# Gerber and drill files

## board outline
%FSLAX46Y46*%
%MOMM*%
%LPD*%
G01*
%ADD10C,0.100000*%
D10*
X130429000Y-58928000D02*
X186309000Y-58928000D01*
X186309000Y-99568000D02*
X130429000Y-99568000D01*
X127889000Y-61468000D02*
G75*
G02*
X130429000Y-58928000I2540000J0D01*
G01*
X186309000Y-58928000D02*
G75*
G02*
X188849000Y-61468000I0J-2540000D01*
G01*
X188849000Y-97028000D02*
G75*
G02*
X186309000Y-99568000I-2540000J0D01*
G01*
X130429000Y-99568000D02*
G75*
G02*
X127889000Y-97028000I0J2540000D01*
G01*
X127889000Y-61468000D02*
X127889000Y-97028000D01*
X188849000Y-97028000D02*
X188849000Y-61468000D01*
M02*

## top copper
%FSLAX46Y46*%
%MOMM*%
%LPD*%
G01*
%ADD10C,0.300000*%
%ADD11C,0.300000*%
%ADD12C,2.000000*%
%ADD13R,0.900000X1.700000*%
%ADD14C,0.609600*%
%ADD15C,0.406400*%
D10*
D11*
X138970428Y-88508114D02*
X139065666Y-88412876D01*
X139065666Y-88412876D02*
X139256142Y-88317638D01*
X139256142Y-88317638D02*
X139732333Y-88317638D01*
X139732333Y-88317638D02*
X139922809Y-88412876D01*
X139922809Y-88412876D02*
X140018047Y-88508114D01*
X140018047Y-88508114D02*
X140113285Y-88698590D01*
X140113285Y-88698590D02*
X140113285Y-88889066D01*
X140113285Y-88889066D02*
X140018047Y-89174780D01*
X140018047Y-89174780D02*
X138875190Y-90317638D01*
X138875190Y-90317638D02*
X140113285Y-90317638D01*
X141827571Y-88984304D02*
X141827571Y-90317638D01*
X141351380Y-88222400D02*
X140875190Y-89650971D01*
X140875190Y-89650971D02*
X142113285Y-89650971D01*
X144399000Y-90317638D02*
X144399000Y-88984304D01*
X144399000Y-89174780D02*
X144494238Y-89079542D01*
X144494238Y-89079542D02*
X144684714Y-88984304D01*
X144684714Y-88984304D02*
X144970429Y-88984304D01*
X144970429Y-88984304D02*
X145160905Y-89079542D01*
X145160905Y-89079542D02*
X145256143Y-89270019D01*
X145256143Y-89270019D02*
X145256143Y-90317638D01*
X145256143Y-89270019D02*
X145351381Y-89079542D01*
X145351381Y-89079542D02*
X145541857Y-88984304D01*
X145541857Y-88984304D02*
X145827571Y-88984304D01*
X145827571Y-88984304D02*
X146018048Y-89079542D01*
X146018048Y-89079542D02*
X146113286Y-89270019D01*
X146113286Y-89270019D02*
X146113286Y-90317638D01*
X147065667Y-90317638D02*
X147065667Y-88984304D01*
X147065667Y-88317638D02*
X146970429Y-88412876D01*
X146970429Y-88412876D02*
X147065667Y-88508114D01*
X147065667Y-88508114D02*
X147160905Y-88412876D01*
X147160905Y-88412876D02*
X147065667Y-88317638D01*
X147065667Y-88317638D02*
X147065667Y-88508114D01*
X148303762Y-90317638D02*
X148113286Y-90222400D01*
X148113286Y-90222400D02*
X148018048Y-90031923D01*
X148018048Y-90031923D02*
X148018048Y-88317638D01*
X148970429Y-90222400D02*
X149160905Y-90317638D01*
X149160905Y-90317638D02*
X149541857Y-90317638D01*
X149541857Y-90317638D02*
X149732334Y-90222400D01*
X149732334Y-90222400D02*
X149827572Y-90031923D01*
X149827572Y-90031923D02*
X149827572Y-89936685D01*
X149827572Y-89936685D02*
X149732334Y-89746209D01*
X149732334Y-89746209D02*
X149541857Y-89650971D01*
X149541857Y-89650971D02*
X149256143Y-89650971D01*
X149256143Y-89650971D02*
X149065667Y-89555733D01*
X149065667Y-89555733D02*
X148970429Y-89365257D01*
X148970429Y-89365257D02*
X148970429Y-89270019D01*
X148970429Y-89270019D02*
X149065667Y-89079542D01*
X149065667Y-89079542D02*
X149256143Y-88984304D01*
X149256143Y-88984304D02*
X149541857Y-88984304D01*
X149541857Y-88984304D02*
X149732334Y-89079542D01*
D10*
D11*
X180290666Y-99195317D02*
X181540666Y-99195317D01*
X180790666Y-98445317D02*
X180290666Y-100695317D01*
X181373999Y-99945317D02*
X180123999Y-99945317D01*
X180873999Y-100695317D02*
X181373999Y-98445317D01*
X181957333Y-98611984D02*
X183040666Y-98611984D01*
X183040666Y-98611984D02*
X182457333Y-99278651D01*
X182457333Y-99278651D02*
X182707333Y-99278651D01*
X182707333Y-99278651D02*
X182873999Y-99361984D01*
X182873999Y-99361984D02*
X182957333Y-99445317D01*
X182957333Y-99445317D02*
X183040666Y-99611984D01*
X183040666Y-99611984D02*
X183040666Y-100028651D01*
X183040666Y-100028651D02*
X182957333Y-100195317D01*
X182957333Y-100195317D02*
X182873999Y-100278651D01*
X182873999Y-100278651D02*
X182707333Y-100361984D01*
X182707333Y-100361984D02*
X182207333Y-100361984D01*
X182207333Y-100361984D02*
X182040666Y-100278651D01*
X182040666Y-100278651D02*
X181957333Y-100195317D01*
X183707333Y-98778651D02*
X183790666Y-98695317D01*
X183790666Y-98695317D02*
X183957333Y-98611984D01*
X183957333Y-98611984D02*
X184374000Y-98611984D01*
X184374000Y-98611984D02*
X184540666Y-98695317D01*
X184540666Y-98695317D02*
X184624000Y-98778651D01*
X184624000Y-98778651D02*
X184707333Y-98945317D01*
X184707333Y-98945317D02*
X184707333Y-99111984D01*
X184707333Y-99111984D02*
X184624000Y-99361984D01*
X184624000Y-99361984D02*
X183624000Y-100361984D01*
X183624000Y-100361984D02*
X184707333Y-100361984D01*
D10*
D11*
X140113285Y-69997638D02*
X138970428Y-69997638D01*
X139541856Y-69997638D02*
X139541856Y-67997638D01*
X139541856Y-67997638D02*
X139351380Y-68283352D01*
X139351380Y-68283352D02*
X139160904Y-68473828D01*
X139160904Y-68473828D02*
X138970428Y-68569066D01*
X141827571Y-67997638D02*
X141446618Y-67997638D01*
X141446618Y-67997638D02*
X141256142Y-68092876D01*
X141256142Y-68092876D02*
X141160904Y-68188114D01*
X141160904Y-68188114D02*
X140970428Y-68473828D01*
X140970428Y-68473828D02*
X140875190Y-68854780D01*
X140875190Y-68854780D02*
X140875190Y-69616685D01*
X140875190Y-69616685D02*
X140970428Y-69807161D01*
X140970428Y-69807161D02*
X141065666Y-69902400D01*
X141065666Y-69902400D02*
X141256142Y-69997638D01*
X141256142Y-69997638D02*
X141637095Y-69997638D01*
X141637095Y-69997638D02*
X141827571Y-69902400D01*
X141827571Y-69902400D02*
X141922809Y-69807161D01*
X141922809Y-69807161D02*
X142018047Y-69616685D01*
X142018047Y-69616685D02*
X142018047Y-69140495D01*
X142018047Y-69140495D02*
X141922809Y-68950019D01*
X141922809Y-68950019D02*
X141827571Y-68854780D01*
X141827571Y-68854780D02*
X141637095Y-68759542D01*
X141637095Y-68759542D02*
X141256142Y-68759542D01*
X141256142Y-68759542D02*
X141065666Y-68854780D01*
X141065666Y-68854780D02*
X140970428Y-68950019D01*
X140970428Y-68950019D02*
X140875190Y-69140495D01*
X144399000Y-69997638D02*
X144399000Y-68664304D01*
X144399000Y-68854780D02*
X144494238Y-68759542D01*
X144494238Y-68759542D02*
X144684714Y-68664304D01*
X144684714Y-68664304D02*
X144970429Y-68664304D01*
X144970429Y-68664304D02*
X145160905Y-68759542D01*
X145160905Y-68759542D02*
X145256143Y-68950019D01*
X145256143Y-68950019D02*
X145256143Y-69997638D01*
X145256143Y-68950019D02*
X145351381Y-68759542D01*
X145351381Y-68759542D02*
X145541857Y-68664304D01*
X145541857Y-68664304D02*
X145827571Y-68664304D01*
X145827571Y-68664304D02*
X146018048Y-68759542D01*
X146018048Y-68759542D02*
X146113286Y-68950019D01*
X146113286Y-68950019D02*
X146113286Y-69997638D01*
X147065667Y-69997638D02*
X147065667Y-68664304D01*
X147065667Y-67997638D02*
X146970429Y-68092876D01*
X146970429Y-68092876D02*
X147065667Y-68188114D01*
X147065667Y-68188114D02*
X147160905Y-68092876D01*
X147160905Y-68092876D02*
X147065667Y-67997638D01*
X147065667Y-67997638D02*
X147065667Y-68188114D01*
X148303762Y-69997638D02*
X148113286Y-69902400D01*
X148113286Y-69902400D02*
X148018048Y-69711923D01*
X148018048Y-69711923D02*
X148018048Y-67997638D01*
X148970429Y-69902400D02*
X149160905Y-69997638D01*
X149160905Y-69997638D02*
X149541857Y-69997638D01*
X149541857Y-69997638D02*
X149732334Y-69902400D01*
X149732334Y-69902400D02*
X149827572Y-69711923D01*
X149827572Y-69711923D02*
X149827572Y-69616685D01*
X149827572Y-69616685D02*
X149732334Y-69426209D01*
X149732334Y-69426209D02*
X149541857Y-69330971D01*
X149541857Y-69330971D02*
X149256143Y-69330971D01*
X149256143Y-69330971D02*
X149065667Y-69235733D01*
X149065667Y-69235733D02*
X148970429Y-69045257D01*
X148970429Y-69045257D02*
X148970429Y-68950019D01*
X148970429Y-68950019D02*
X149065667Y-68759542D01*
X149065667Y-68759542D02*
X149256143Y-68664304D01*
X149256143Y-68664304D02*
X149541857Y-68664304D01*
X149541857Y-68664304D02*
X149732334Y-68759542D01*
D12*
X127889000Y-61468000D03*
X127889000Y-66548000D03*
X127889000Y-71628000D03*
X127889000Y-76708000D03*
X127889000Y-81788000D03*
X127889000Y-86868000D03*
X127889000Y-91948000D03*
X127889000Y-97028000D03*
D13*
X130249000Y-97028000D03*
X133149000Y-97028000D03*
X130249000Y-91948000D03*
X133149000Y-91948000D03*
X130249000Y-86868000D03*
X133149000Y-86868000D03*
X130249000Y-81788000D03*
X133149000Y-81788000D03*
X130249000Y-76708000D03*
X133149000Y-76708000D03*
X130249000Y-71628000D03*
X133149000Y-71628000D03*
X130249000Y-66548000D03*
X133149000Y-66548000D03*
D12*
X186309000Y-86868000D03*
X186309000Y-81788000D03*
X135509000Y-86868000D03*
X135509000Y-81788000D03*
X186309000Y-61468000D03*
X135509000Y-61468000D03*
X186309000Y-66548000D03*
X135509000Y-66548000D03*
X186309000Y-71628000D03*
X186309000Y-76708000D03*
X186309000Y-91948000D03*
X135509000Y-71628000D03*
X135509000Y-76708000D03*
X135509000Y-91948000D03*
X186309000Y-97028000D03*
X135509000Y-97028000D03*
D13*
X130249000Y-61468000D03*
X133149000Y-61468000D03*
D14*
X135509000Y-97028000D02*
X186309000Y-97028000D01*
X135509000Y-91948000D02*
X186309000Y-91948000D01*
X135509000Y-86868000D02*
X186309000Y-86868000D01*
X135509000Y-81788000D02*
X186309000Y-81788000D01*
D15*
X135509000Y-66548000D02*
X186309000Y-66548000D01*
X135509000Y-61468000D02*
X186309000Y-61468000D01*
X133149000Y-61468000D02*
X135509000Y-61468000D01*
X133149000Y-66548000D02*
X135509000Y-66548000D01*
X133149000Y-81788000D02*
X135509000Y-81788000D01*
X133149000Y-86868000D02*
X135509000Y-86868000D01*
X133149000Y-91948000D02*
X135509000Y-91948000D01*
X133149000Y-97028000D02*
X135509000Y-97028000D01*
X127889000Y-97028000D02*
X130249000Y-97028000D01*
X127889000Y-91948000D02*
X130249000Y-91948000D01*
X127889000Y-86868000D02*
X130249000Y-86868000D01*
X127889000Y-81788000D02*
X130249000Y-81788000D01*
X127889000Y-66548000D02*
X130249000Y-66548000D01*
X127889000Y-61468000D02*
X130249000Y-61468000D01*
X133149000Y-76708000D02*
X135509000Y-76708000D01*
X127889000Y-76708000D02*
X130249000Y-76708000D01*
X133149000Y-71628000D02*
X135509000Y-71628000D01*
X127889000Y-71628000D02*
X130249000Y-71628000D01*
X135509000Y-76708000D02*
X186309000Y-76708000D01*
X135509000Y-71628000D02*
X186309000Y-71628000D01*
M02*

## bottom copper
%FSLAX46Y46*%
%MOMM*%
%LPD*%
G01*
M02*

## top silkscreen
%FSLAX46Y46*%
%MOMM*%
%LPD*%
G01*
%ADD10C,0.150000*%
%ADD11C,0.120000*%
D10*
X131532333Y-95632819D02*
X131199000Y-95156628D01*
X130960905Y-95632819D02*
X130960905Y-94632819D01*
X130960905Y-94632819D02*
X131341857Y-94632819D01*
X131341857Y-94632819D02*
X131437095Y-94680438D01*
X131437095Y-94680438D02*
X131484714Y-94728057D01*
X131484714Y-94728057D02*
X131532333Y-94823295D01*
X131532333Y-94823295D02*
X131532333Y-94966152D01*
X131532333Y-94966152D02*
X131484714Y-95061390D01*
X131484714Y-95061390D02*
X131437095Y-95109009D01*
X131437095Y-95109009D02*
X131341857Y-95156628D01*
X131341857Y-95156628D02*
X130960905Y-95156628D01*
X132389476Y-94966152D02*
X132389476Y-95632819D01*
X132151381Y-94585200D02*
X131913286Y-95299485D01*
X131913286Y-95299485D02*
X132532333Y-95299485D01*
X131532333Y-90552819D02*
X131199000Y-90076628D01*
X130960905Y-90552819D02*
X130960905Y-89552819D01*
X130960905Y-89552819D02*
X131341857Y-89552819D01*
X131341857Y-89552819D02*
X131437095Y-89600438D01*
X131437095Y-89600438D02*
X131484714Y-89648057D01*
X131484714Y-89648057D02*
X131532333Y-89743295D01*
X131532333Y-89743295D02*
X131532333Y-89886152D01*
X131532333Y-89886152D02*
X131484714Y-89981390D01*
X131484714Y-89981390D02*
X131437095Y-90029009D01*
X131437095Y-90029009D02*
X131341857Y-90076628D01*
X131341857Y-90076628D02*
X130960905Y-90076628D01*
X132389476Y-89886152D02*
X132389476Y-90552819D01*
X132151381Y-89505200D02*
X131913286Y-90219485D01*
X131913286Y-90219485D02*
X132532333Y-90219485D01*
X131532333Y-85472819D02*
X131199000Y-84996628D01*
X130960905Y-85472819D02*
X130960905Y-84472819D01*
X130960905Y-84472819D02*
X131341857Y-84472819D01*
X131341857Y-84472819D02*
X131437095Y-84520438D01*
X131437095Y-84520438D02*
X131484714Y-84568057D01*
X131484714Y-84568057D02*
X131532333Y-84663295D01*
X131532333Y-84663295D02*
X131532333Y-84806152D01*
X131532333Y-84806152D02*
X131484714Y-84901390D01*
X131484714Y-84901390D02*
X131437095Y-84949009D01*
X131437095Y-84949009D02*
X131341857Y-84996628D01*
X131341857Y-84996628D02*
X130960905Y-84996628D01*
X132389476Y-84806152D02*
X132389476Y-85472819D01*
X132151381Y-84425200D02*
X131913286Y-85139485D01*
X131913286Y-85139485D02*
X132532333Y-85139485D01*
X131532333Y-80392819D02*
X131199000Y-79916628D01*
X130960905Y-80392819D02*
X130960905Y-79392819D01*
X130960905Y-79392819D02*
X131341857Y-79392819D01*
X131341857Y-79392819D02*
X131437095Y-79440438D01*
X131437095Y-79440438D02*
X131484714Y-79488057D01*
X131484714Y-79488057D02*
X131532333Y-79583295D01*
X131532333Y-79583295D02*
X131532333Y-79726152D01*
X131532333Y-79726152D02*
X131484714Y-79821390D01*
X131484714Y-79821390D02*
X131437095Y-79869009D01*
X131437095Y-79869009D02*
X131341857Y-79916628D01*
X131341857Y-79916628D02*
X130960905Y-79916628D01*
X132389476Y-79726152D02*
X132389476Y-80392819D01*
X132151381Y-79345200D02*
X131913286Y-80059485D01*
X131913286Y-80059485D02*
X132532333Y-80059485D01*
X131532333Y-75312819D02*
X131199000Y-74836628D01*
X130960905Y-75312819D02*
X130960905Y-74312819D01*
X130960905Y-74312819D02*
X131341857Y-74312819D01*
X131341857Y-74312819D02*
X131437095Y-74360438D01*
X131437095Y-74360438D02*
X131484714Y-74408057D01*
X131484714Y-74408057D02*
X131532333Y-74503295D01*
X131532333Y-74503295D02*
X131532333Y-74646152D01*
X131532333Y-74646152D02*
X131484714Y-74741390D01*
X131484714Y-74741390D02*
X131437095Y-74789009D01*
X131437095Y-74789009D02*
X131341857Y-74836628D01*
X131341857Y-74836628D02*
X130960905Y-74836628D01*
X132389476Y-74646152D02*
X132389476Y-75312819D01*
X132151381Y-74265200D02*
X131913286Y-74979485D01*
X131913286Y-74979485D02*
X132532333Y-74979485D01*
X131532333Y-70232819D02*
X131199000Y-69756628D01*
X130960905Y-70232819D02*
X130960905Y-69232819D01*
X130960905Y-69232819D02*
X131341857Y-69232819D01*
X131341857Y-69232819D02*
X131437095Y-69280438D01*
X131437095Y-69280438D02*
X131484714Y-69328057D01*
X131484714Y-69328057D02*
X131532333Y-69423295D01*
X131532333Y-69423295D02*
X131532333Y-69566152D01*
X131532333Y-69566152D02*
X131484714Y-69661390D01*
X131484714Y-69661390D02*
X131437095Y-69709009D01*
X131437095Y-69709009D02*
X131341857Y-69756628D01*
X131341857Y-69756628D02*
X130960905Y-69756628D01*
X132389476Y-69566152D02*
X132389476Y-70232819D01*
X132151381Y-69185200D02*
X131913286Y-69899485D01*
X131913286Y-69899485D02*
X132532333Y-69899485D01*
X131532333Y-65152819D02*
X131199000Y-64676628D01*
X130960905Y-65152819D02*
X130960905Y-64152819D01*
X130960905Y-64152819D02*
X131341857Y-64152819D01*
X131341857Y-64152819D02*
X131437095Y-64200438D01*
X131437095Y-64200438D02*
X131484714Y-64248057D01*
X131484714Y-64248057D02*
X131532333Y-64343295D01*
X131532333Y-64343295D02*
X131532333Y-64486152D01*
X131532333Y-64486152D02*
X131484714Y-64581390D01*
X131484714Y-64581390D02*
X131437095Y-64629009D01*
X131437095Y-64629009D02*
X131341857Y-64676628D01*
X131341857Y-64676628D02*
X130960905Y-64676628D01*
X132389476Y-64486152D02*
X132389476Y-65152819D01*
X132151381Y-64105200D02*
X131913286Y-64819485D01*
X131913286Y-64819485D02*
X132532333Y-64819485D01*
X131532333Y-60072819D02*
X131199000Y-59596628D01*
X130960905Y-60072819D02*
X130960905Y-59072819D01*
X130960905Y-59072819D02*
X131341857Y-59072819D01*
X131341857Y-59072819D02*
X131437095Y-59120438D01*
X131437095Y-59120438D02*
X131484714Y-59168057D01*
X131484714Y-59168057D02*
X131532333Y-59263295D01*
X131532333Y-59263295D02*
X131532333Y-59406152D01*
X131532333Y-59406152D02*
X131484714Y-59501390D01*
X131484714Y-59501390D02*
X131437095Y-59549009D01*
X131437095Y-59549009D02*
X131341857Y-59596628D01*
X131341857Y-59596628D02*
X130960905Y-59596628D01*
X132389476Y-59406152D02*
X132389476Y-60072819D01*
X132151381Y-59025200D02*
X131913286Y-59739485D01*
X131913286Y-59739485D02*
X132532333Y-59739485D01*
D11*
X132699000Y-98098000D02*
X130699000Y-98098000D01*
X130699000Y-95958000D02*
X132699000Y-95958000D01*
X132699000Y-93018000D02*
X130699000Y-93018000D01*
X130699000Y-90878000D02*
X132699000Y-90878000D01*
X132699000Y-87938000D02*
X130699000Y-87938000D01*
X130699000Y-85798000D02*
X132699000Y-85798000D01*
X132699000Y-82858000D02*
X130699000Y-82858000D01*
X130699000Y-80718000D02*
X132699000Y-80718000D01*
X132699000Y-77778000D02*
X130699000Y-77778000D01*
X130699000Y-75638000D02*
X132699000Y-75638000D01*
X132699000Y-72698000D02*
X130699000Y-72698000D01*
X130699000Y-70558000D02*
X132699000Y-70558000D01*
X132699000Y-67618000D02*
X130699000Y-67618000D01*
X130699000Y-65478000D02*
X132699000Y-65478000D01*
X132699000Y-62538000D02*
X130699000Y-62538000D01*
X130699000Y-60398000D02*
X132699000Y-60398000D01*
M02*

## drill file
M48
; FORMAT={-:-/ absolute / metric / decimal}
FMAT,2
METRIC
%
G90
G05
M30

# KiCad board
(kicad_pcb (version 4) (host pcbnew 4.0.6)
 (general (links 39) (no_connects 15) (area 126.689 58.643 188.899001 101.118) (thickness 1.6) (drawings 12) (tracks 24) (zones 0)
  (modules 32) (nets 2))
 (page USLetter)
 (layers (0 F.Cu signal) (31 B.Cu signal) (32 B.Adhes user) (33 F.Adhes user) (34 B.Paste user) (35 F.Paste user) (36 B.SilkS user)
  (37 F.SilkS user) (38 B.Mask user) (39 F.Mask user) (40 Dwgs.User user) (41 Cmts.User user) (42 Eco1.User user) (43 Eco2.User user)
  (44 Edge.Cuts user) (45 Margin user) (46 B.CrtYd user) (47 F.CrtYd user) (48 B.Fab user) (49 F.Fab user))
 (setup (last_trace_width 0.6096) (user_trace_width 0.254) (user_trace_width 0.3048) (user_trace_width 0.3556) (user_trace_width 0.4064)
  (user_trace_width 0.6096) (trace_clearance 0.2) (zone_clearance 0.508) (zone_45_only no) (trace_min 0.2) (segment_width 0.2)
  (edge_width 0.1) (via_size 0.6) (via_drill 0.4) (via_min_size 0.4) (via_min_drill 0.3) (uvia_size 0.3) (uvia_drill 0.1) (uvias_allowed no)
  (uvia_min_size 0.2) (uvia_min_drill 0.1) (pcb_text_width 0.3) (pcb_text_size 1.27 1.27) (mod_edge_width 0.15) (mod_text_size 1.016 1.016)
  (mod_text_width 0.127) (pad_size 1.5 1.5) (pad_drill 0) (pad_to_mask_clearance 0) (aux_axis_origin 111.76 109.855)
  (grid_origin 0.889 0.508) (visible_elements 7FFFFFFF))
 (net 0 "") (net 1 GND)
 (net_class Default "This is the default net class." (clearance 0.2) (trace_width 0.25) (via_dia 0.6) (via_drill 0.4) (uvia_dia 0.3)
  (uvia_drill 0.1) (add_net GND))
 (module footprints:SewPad (layer F.Cu) (at 127.889 61.468 90)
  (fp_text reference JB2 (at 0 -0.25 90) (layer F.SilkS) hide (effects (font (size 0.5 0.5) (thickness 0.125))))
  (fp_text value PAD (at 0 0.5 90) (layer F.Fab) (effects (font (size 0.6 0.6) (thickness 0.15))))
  (pad 1 smd circle (at 0 0 90) (size 2 2) (layers F.Cu F.Mask) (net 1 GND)))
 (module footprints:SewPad (layer F.Cu) (at 127.889 66.548 90)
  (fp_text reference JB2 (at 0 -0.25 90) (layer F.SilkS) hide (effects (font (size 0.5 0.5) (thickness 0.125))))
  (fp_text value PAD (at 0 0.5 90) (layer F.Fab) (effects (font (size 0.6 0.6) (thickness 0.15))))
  (pad 1 smd circle (at 0 0 90) (size 2 2) (layers F.Cu F.Mask) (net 1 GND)))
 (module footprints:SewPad (layer F.Cu) (at 127.889 71.628 90)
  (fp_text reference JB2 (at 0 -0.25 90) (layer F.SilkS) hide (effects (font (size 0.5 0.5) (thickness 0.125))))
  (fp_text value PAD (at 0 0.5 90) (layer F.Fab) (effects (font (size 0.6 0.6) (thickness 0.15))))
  (pad 1 smd circle (at 0 0 90) (size 2 2) (layers F.Cu F.Mask) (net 1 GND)))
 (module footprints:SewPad (layer F.Cu) (at 127.889 76.708 90)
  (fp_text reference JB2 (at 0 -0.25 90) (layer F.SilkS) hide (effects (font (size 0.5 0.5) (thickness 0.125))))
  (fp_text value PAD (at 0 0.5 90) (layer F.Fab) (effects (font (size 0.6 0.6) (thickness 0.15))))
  (pad 1 smd circle (at 0 0 90) (size 2 2) (layers F.Cu F.Mask) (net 1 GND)))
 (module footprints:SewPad (layer F.Cu) (at 127.889 81.788 90)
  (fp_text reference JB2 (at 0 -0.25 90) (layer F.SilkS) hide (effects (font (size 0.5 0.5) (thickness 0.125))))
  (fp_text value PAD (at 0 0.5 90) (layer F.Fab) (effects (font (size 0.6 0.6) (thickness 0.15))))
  (pad 1 smd circle (at 0 0 90) (size 2 2) (layers F.Cu F.Mask) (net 1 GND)))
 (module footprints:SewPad (layer F.Cu) (at 127.889 86.868 90)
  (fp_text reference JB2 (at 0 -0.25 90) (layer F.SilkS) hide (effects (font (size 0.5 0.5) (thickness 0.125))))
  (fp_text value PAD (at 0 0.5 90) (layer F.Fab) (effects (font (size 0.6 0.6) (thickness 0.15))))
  (pad 1 smd circle (at 0 0 90) (size 2 2) (layers F.Cu F.Mask) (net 1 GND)))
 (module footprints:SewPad (layer F.Cu) (at 127.889 91.948 90)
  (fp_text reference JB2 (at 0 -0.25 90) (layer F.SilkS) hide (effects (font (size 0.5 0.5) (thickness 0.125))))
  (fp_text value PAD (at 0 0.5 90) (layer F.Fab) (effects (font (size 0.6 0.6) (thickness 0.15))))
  (pad 1 smd circle (at 0 0 90) (size 2 2) (layers F.Cu F.Mask) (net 1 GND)))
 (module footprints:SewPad (layer F.Cu) (at 127.889 97.028 90)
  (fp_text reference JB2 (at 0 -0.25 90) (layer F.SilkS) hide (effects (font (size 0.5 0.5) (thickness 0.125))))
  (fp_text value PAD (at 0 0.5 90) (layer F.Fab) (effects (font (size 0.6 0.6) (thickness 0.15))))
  (pad 1 smd circle (at 0 0 90) (size 2 2) (layers F.Cu F.Mask) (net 1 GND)))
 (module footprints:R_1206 (layer F.Cu) (at 131.699 97.028)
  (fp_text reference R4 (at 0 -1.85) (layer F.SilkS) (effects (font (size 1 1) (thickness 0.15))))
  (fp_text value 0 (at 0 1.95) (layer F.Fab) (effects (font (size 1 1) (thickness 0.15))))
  (fp_line (start 1 1.07) (end -1 1.07) (layer F.SilkS) (width 0.12))
  (fp_line (start -1 -1.07) (end 1 -1.07) (layer F.SilkS) (width 0.12))
  (pad 1 smd rect (at -1.45 0) (size 0.9 1.7) (layers F.Cu F.Paste F.Mask) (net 1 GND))
  (pad 2 smd rect (at 1.45 0) (size 0.9 1.7) (layers F.Cu F.Paste F.Mask) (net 1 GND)))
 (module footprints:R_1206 (layer F.Cu) (at 131.699 91.948)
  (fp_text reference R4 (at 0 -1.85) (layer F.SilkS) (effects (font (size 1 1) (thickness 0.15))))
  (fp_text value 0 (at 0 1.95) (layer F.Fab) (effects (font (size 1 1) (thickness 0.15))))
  (fp_line (start 1 1.07) (end -1 1.07) (layer F.SilkS) (width 0.12))
  (fp_line (start -1 -1.07) (end 1 -1.07) (layer F.SilkS) (width 0.12))
  (pad 1 smd rect (at -1.45 0) (size 0.9 1.7) (layers F.Cu F.Paste F.Mask) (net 1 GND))
  (pad 2 smd rect (at 1.45 0) (size 0.9 1.7) (layers F.Cu F.Paste F.Mask) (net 1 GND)))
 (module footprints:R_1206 (layer F.Cu) (at 131.699 86.868)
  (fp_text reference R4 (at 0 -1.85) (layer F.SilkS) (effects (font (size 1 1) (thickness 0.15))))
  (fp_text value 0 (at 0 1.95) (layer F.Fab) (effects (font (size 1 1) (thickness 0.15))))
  (fp_line (start 1 1.07) (end -1 1.07) (layer F.SilkS) (width 0.12))
  (fp_line (start -1 -1.07) (end 1 -1.07) (layer F.SilkS) (width 0.12))
  (pad 1 smd rect (at -1.45 0) (size 0.9 1.7) (layers F.Cu F.Paste F.Mask) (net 1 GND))
  (pad 2 smd rect (at 1.45 0) (size 0.9 1.7) (layers F.Cu F.Paste F.Mask) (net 1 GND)))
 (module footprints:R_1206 (layer F.Cu) (at 131.699 81.788)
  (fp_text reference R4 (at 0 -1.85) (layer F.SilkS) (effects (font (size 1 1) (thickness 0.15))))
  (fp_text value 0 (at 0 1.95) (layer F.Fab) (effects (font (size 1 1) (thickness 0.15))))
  (fp_line (start 1 1.07) (end -1 1.07) (layer F.SilkS) (width 0.12))
  (fp_line (start -1 -1.07) (end 1 -1.07) (layer F.SilkS) (width 0.12))
  (pad 1 smd rect (at -1.45 0) (size 0.9 1.7) (layers F.Cu F.Paste F.Mask) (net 1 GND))
  (pad 2 smd rect (at 1.45 0) (size 0.9 1.7) (layers F.Cu F.Paste F.Mask) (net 1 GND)))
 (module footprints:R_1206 (layer F.Cu) (at 131.699 76.708)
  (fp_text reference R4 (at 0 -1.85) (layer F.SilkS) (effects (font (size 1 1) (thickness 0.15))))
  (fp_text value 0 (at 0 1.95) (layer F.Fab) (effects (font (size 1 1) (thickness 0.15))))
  (fp_line (start 1 1.07) (end -1 1.07) (layer F.SilkS) (width 0.12))
  (fp_line (start -1 -1.07) (end 1 -1.07) (layer F.SilkS) (width 0.12))
  (pad 1 smd rect (at -1.45 0) (size 0.9 1.7) (layers F.Cu F.Paste F.Mask) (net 1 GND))
  (pad 2 smd rect (at 1.45 0) (size 0.9 1.7) (layers F.Cu F.Paste F.Mask) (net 1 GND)))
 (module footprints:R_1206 (layer F.Cu) (at 131.699 71.628)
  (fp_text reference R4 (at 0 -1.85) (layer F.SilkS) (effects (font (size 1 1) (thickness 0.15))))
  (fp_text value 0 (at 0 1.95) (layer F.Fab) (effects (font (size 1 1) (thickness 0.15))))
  (fp_line (start 1 1.07) (end -1 1.07) (layer F.SilkS) (width 0.12))
  (fp_line (start -1 -1.07) (end 1 -1.07) (layer F.SilkS) (width 0.12))
  (pad 1 smd rect (at -1.45 0) (size 0.9 1.7) (layers F.Cu F.Paste F.Mask) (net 1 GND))
  (pad 2 smd rect (at 1.45 0) (size 0.9 1.7) (layers F.Cu F.Paste F.Mask) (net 1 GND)))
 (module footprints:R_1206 (layer F.Cu) (at 131.699 66.548)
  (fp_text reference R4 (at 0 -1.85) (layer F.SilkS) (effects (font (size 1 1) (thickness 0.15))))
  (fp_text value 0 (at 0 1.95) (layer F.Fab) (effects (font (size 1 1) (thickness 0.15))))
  (fp_line (start 1 1.07) (end -1 1.07) (layer F.SilkS) (width 0.12))
  (fp_line (start -1 -1.07) (end 1 -1.07) (layer F.SilkS) (width 0.12))
  (pad 1 smd rect (at -1.45 0) (size 0.9 1.7) (layers F.Cu F.Paste F.Mask) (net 1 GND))
  (pad 2 smd rect (at 1.45 0) (size 0.9 1.7) (layers F.Cu F.Paste F.Mask) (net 1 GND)))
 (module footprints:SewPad (layer F.Cu) (at 186.309 86.868 90)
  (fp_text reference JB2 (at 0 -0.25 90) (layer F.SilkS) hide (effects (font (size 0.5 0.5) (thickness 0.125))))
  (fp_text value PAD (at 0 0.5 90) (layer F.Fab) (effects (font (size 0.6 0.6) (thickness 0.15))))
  (pad 1 smd circle (at 0 0 90) (size 2 2) (layers F.Cu F.Mask) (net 1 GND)))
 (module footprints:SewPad (layer F.Cu) (at 186.309 81.788 90)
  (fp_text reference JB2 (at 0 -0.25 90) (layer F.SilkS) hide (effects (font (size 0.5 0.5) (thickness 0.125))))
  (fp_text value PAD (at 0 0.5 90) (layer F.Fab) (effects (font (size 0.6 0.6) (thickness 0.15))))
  (pad 1 smd circle (at 0 0 90) (size 2 2) (layers F.Cu F.Mask) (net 1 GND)))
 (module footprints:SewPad (layer F.Cu) (at 135.509 86.868 90)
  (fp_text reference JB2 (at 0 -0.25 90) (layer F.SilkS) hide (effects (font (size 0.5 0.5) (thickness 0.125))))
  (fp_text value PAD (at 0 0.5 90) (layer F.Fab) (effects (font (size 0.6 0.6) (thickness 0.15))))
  (pad 1 smd circle (at 0 0 90) (size 2 2) (layers F.Cu F.Mask) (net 1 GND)))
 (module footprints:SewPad (layer F.Cu) (at 135.509 81.788 90)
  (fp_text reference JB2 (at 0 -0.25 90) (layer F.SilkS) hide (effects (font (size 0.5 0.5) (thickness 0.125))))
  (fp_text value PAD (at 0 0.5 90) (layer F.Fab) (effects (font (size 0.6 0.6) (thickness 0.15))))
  (pad 1 smd circle (at 0 0 90) (size 2 2) (layers F.Cu F.Mask) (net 1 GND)))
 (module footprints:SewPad (layer F.Cu) (at 186.309 61.468 90)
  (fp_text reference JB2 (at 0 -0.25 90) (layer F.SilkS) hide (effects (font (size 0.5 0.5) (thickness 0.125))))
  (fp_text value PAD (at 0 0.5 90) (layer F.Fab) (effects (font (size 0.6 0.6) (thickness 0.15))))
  (pad 1 smd circle (at 0 0 90) (size 2 2) (layers F.Cu F.Mask) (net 1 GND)))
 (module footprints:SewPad (layer F.Cu) (at 135.509 61.468 90)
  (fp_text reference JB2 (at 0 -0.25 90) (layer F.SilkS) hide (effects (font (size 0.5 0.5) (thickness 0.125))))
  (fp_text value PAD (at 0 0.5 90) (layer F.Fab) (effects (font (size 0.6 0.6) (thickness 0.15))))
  (pad 1 smd circle (at 0 0 90) (size 2 2) (layers F.Cu F.Mask) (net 1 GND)))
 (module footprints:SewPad (layer F.Cu) (at 186.309 66.548 90)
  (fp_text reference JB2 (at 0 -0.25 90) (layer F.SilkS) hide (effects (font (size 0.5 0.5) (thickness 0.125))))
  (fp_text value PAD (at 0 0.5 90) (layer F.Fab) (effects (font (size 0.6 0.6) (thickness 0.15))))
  (pad 1 smd circle (at 0 0 90) (size 2 2) (layers F.Cu F.Mask) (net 1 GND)))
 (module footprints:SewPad (layer F.Cu) (at 135.509 66.548 90)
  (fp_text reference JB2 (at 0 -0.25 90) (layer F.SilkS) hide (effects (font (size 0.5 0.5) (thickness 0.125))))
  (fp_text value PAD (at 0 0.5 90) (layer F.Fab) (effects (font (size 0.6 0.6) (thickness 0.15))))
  (pad 1 smd circle (at 0 0 90) (size 2 2) (layers F.Cu F.Mask) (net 1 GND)))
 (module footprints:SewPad (layer F.Cu) (at 186.309 71.628 90)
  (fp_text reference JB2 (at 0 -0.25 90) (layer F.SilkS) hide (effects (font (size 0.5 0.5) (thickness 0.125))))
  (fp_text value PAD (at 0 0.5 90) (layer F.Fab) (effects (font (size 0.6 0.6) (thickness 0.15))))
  (pad 1 smd circle (at 0 0 90) (size 2 2) (layers F.Cu F.Mask) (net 1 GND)))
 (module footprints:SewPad (layer F.Cu) (at 186.309 76.708 90)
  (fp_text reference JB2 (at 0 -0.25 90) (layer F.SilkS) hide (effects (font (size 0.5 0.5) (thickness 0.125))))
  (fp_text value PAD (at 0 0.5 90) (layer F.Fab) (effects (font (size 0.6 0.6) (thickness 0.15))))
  (pad 1 smd circle (at 0 0 90) (size 2 2) (layers F.Cu F.Mask) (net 1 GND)))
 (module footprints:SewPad (layer F.Cu) (at 186.309 91.948 90)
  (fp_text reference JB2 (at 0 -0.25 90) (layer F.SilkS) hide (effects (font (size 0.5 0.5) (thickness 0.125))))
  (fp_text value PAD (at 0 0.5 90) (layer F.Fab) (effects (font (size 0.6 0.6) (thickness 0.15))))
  (pad 1 smd circle (at 0 0 90) (size 2 2) (layers F.Cu F.Mask) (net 1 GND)))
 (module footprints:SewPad (layer F.Cu) (at 135.509 71.628 90)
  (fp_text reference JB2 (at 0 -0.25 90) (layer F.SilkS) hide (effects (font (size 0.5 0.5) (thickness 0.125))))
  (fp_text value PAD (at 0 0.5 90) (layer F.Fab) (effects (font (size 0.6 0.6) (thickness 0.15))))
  (pad 1 smd circle (at 0 0 90) (size 2 2) (layers F.Cu F.Mask) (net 1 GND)))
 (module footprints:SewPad (layer F.Cu) (at 135.509 76.708 90)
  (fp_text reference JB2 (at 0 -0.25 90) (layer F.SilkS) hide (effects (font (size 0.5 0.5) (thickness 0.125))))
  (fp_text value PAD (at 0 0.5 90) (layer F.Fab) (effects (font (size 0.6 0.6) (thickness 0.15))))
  (pad 1 smd circle (at 0 0 90) (size 2 2) (layers F.Cu F.Mask) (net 1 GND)))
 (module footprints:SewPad (layer F.Cu) (at 135.509 91.948 90)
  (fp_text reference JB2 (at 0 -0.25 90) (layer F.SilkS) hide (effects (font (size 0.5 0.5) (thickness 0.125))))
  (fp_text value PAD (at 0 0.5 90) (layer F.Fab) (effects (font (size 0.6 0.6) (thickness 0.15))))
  (pad 1 smd circle (at 0 0 90) (size 2 2) (layers F.Cu F.Mask) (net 1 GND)))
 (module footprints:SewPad (layer F.Cu) (at 186.309 97.028 90)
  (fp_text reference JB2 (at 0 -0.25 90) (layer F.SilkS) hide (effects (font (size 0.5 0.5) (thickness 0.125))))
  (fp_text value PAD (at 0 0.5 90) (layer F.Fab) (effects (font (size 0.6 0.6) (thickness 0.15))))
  (pad 1 smd circle (at 0 0 90) (size 2 2) (layers F.Cu F.Mask) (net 1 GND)))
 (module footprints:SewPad (layer F.Cu) (at 135.509 97.028 90)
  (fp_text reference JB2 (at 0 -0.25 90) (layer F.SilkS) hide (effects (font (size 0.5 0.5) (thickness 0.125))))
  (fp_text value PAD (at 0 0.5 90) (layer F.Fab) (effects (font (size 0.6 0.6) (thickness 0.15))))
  (pad 1 smd circle (at 0 0 90) (size 2 2) (layers F.Cu F.Mask) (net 1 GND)))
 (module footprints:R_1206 (layer F.Cu) (at 131.699 61.468)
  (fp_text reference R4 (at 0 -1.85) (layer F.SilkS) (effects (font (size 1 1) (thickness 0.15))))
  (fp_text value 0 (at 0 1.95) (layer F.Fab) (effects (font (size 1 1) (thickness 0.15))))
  (fp_line (start 1 1.07) (end -1 1.07) (layer F.SilkS) (width 0.12))
  (fp_line (start -1 -1.07) (end 1 -1.07) (layer F.SilkS) (width 0.12))
  (pad 1 smd rect (at -1.45 0) (size 0.9 1.7) (layers F.Cu F.Paste F.Mask) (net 1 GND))
  (pad 2 smd rect (at 1.45 0) (size 0.9 1.7) (layers F.Cu F.Paste F.Mask) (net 1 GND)))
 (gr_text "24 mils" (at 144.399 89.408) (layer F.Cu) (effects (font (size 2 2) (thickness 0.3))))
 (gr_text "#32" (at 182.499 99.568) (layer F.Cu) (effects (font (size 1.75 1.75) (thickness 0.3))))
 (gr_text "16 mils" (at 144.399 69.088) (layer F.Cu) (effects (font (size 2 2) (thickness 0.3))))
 (gr_line (start 130.429 58.928) (end 186.309 58.928) (angle 90) (layer Edge.Cuts) (width 0.1))
 (gr_line (start 186.309 99.568) (end 130.429 99.568) (angle 90) (layer Edge.Cuts) (width 0.1))
 (gr_arc (start 130.429 61.468) (end 127.889 61.468) (angle 90) (layer Edge.Cuts) (width 0.1))
 (gr_arc (start 186.309 61.468) (end 186.309 58.928) (angle 90) (layer Edge.Cuts) (width 0.1))
 (gr_arc (start 186.309 97.028) (end 188.849 97.028) (angle 90) (layer Edge.Cuts) (width 0.1))
 (gr_arc (start 130.429 97.028) (end 130.429 99.568) (angle 90) (layer Edge.Cuts) (width 0.1))
 (gr_line (start 127.889 61.468) (end 127.889 97.028) (angle 90) (layer Edge.Cuts) (width 0.1))
 (gr_line (start 188.849 97.028) (end 188.849 61.468) (angle 90) (layer Edge.Cuts) (width 0.1))
 (segment (start 135.509 97.028) (end 186.309 97.028) (width 0.6096) (layer F.Cu) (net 1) (status C00000))
 (segment (start 135.509 91.948) (end 186.309 91.948) (width 0.6096) (layer F.Cu) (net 1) (status C00000))
 (segment (start 135.509 86.868) (end 186.309 86.868) (width 0.6096) (layer F.Cu) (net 1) (status C00000))
 (segment (start 135.509 81.788) (end 186.309 81.788) (width 0.6096) (layer F.Cu) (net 1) (status C00000))
 (segment (start 135.509 66.548) (end 186.309 66.548) (width 0.4064) (layer F.Cu) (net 1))
 (segment (start 135.509 61.468) (end 186.309 61.468) (width 0.4064) (layer F.Cu) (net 1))
 (segment (start 133.149 61.468) (end 135.509 61.468) (width 0.4064) (layer F.Cu) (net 1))
 (segment (start 133.149 66.548) (end 135.509 66.548) (width 0.4064) (layer F.Cu) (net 1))
 (segment (start 133.149 81.788) (end 135.509 81.788) (width 0.4064) (layer F.Cu) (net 1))
 (segment (start 133.149 86.868) (end 135.509 86.868) (width 0.4064) (layer F.Cu) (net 1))
 (segment (start 133.149 91.948) (end 135.509 91.948) (width 0.4064) (layer F.Cu) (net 1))
 (segment (start 133.149 97.028) (end 135.509 97.028) (width 0.4064) (layer F.Cu) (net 1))
 (segment (start 127.889 97.028) (end 130.249 97.028) (width 0.4064) (layer F.Cu) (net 1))
 (segment (start 127.889 91.948) (end 130.249 91.948) (width 0.4064) (layer F.Cu) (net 1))
 (segment (start 127.889 86.868) (end 130.249 86.868) (width 0.4064) (layer F.Cu) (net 1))
 (segment (start 127.889 81.788) (end 130.249 81.788) (width 0.4064) (layer F.Cu) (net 1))
 (segment (start 127.889 66.548) (end 130.249 66.548) (width 0.4064) (layer F.Cu) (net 1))
 (segment (start 127.889 61.468) (end 130.249 61.468) (width 0.4064) (layer F.Cu) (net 1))
 (segment (start 133.149 76.708) (end 135.509 76.708) (width 0.4064) (layer F.Cu) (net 1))
 (segment (start 127.889 76.708) (end 130.249 76.708) (width 0.4064) (layer F.Cu) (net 1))
 (segment (start 133.149 71.628) (end 135.509 71.628) (width 0.4064) (layer F.Cu) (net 1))
 (segment (start 127.889 71.628) (end 130.249 71.628) (width 0.4064) (layer F.Cu) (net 1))
 (segment (start 135.509 76.708) (end 186.309 76.708) (width 0.4064) (layer F.Cu) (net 1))
 (segment (start 135.509 71.628) (end 186.309 71.628) (width 0.4064) (layer F.Cu) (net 1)))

